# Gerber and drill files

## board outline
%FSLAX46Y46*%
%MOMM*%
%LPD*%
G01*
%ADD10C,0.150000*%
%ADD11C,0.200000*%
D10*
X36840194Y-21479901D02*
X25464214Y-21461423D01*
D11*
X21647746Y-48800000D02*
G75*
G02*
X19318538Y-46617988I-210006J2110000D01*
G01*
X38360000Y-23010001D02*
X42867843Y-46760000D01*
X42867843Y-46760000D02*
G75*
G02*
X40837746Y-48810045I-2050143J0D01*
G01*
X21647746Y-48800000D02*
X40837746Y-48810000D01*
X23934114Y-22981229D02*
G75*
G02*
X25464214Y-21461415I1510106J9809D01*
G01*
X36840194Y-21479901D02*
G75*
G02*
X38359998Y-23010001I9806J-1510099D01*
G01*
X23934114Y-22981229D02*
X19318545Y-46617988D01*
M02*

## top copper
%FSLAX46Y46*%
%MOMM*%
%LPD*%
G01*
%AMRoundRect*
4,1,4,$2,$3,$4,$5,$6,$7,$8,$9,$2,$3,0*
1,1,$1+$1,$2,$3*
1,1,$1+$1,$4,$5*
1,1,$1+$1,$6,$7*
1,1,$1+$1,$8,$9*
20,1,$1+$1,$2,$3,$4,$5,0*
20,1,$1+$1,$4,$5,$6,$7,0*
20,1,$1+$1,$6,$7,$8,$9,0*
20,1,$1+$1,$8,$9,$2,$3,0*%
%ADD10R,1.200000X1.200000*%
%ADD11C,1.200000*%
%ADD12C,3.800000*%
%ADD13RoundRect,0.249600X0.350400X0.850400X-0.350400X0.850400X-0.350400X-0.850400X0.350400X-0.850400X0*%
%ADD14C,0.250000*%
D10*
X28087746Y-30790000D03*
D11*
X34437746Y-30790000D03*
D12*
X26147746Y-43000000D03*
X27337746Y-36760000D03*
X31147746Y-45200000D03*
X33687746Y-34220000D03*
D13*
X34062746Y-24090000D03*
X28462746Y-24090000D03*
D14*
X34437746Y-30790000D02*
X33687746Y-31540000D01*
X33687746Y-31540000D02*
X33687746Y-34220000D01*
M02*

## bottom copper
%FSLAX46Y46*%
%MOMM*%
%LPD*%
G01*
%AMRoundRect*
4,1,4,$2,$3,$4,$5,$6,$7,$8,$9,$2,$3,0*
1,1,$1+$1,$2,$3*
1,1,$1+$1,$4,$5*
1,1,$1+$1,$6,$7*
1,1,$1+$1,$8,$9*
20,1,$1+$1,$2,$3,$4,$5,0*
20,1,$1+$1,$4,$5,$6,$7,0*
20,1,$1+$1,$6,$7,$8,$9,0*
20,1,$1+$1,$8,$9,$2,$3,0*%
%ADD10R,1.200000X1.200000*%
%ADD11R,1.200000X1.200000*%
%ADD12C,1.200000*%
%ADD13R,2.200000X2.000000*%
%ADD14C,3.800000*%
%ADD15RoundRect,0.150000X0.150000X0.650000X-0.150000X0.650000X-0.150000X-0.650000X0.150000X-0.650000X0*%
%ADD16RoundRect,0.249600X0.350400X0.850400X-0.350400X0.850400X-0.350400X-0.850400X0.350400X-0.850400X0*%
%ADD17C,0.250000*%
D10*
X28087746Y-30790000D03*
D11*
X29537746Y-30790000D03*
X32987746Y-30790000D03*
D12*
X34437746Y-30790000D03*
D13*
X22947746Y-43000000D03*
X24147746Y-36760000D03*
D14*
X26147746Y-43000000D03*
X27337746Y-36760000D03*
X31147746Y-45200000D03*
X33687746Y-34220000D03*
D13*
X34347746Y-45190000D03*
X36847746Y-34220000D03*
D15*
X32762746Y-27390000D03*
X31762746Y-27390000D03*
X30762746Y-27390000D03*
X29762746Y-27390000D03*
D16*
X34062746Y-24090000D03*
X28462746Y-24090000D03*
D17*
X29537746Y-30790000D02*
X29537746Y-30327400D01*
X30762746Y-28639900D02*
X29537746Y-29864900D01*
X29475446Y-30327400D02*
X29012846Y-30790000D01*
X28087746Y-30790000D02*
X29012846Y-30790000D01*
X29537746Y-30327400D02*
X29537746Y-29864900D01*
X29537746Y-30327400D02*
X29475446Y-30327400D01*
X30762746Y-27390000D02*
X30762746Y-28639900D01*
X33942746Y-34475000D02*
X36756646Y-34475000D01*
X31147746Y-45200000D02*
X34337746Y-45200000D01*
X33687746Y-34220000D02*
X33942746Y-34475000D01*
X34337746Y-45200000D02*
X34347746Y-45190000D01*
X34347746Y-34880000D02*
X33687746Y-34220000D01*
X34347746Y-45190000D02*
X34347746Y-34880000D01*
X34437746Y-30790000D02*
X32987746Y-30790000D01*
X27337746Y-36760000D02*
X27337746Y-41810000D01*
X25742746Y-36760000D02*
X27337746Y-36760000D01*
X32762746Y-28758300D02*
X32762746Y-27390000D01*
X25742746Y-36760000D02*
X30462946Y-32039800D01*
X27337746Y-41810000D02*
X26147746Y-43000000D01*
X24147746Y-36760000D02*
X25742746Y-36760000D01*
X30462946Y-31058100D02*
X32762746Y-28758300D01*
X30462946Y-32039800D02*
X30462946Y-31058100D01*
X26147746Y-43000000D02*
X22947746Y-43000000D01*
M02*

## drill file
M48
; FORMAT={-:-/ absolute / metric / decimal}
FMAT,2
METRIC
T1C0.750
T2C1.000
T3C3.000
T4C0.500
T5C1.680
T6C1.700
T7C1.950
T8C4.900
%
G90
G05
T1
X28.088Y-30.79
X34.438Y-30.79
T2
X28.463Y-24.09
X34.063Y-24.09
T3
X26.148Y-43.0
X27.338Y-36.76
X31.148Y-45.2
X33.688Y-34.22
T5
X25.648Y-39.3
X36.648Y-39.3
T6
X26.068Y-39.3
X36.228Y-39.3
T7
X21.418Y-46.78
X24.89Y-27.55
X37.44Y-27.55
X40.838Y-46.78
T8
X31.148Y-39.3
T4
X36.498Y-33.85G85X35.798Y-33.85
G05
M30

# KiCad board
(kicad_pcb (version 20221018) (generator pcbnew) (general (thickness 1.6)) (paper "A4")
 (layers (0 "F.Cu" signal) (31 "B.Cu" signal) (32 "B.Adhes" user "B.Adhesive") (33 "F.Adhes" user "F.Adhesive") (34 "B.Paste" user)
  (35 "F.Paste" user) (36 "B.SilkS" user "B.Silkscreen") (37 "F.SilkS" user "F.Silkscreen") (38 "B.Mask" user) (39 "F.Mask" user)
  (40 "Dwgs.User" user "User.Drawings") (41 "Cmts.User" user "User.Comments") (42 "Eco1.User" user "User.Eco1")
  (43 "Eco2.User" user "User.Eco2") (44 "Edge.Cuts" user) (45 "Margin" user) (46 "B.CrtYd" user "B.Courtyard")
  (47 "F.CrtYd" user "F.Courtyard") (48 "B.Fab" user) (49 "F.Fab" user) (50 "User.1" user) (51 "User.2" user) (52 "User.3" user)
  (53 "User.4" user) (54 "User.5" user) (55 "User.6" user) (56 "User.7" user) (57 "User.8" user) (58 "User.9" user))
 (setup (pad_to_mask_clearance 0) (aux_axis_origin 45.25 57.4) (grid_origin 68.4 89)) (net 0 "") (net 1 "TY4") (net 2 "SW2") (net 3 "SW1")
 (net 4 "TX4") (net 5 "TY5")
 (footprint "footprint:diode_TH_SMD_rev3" (layer "F.Cu") (at 31.262746 30.79)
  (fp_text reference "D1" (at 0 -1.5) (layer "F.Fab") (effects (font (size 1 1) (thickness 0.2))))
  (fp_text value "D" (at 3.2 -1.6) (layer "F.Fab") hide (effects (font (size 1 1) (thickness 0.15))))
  (pad "1" thru_hole rect (at -3.175 0) (size 1.2 1.2) (drill 0.75) (layers "*.Cu" "B.Mask") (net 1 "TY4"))
  (pad "1" smd rect (at -1.725 0) (size 1.2 1.2) (layers "B.Cu" "B.Paste" "B.Mask") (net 1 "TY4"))
  (pad "2" smd rect (at 1.725 0) (size 1.2 1.2) (layers "B.Cu" "B.Paste" "B.Mask") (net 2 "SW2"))
  (pad "2" thru_hole circle (at 3.175 0) (size 1.2 1.2) (drill 0.75) (layers "*.Cu" "B.Mask") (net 2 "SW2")))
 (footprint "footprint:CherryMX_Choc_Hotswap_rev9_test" (layer "F.Cu") (at 31.147746 39.3)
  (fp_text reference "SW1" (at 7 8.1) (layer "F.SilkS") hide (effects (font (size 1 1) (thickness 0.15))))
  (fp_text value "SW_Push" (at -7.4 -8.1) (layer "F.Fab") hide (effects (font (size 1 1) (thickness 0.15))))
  (pad "" np_thru_hole circle (at -5.5 0 90) (size 1.68 1.68) (drill 1.68) (layers "*.Cu" "*.Mask"))
  (pad "" np_thru_hole circle (at -5.08 0) (size 1.7 1.7) (drill 1.7) (layers "*.Cu" "*.Mask"))
  (pad "" np_thru_hole circle (at 0 0 90) (size 4.9 4.9) (drill 4.9) (layers "*.Cu" "*.Mask"))
  (pad "" np_thru_hole oval (at 5 -5.45 180) (size 1.2 0.5) (drill oval 1.2 0.5) (layers "*.Cu" "*.Mask"))
  (pad "" np_thru_hole circle (at 5.08 0) (size 1.7 1.7) (drill 1.7) (layers "*.Cu" "*.Mask"))
  (pad "" np_thru_hole circle (at 5.5 0 90) (size 1.68 1.68) (drill 1.68) (layers "*.Cu" "*.Mask"))
  (pad "1" smd rect (at -8.2 3.7) (size 2.2 2) (layers "B.Cu" "B.Paste" "B.Mask") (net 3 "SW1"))
  (pad "1" smd rect (at -7 -2.54) (size 2.2 2) (layers "B.Cu" "B.Paste" "B.Mask") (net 3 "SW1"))
  (pad "1" thru_hole circle (at -5 3.7 90) (size 3.8 3.8) (drill 3) (layers "*.Cu" "B.Mask") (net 3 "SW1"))
  (pad "1" thru_hole circle (at -3.81 -2.54 180) (size 3.8 3.8) (drill 3) (layers "*.Cu" "B.Mask") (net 3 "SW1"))
  (pad "2" thru_hole circle (at 0 5.9 90) (size 3.8 3.8) (drill 3) (layers "*.Cu" "B.Mask") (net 2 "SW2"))
  (pad "2" thru_hole circle (at 2.54 -5.08 180) (size 3.8 3.8) (drill 3) (layers "*.Cu" "B.Mask") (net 2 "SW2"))
  (pad "2" smd rect (at 3.2 5.89) (size 2.2 2) (layers "B.Cu" "B.Paste" "B.Mask") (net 2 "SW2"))
  (pad "2" smd rect (at 5.7 -5.08) (size 2.2 2) (layers "B.Cu" "B.Paste" "B.Mask") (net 2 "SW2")))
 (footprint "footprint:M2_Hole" (layer "F.Cu") (at 40.837746 46.78)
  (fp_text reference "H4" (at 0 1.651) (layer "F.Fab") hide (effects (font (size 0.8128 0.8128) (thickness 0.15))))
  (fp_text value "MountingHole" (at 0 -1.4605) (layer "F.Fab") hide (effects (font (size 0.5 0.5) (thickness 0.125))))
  (pad "" np_thru_hole circle (at 0 0) (size 1.95 1.95) (drill 1.95) (layers "F&B.Cu" "*.Mask")))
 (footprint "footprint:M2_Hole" (layer "F.Cu") (at 21.417746 46.78)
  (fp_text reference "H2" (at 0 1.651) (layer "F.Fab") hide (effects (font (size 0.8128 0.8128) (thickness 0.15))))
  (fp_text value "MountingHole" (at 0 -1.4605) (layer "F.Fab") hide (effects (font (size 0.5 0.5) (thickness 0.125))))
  (pad "" np_thru_hole circle (at 0 0) (size 1.95 1.95) (drill 1.95) (layers "F&B.Cu" "*.Mask")))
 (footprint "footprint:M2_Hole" (layer "F.Cu") (at 24.89 27.55)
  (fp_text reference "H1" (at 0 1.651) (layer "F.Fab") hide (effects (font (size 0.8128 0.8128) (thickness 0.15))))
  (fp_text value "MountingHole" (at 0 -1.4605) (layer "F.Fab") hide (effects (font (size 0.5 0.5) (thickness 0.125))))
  (pad "" np_thru_hole circle (at 0 0) (size 1.95 1.95) (drill 1.95) (layers "F&B.Cu" "*.Mask")))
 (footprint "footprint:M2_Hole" (layer "F.Cu") (at 37.44 27.55)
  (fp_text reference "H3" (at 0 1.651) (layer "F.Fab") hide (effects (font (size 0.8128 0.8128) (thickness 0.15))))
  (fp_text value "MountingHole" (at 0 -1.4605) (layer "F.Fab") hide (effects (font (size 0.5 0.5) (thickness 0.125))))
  (pad "" np_thru_hole circle (at 0 0) (size 1.95 1.95) (drill 1.95) (layers "F&B.Cu" "*.Mask")))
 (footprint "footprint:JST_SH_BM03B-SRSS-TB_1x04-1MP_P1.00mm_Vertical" (layer "B.Cu") (at 31.262746 25.59 180)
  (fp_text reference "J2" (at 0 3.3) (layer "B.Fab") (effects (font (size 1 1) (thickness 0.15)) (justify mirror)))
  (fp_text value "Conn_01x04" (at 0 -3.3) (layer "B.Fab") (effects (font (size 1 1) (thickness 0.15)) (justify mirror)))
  (pad "1" smd roundrect (at -1.5 -1.8 180) (size 0.6 1.6) (layers "B.Cu" "B.Paste" "B.Mask") (roundrect_rratio 0.25) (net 3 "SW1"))
  (pad "2" smd roundrect (at -0.5 -1.8 180) (size 0.6 1.6) (layers "B.Cu" "B.Paste" "B.Mask") (roundrect_rratio 0.25) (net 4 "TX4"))
  (pad "3" smd roundrect (at 0.5 -1.8 180) (size 0.6 1.6) (layers "B.Cu" "B.Paste" "B.Mask") (roundrect_rratio 0.25) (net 1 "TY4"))
  (pad "4" smd roundrect (at 1.5 -1.8 180) (size 0.6 1.6) (layers "B.Cu" "B.Paste" "B.Mask") (roundrect_rratio 0.25) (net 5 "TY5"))
  (pad "MP" thru_hole roundrect (at -2.8 1.5 180) (size 1.2 2.2) (drill 1) (layers "*.Cu" "*.Mask") (roundrect_rratio 0.208))
  (pad "MP" thru_hole roundrect (at 2.8 1.5 180) (size 1.2 2.2) (drill 1) (layers "*.Cu" "*.Mask") (roundrect_rratio 0.208)))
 (gr_line (start 36.840194 21.479901) (end 25.464214 21.461423) (stroke (width 0.15) (type default)) (layer "Edge.Cuts"))
 (gr_arc (start 21.647746 48.8) (mid 19.988071 48.237464) (end 19.318545 46.617988) (stroke (width 0.2) (type default)) (layer "Edge.Cuts"))
 (gr_line (start 38.36 23.010001) (end 42.867843 46.76) (stroke (width 0.2) (type default)) (layer "Edge.Cuts"))
 (gr_arc (start 42.867843 46.76) (mid 42.274437 48.202549) (end 40.837746 48.809999) (stroke (width 0.2) (type default)) (layer "Edge.Cuts"))
 (gr_line (start 21.647746 48.8) (end 40.837746 48.81) (stroke (width 0.2) (type default)) (layer "Edge.Cuts"))
 (gr_arc (start 23.934114 22.981229) (mid 24.38 21.900001) (end 25.464214 21.461423) (stroke (width 0.2) (type default)) (layer "Edge.Cuts"))
 (gr_arc (start 36.840194 21.479901) (mid 37.921422 21.925787) (end 38.36 23.010001) (stroke (width 0.2) (type default)) (layer "Edge.Cuts"))
 (gr_line (start 23.934114 22.981229) (end 19.318545 46.617988) (stroke (width 0.2) (type default)) (layer "Edge.Cuts"))
 (segment (start 29.537746 30.79) (end 29.537746 30.3274) (width 0.25) (layer "B.Cu") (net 1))
 (segment (start 30.762746 28.6399) (end 29.537746 29.8649) (width 0.25) (layer "B.Cu") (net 1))
 (segment (start 29.475446 30.3274) (end 29.012846 30.79) (width 0.25) (layer "B.Cu") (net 1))
 (segment (start 28.087746 30.79) (end 29.012846 30.79) (width 0.25) (layer "B.Cu") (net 1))
 (segment (start 29.537746 30.3274) (end 29.537746 29.8649) (width 0.25) (layer "B.Cu") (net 1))
 (segment (start 29.537746 30.3274) (end 29.475446 30.3274) (width 0.25) (layer "B.Cu") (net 1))
 (segment (start 30.762746 27.39) (end 30.762746 28.6399) (width 0.25) (layer "B.Cu") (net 1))
 (segment (start 34.437746 30.79) (end 33.687746 31.54) (width 0.25) (layer "F.Cu") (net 2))
 (segment (start 33.687746 31.54) (end 33.687746 34.22) (width 0.25) (layer "F.Cu") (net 2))
 (segment (start 33.942746 34.475) (end 36.756646 34.475) (width 0.25) (layer "B.Cu") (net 2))
 (segment (start 31.147746 45.2) (end 34.337746 45.2) (width 0.25) (layer "B.Cu") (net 2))
 (segment (start 33.687746 34.22) (end 33.942746 34.475) (width 0.25) (layer "B.Cu") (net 2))
 (segment (start 34.337746 45.2) (end 34.347746 45.19) (width 0.25) (layer "B.Cu") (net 2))
 (segment (start 34.347746 34.88) (end 33.687746 34.22) (width 0.25) (layer "B.Cu") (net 2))
 (segment (start 34.347746 45.19) (end 34.347746 34.88) (width 0.25) (layer "B.Cu") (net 2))
 (segment (start 34.437746 30.79) (end 32.987746 30.79) (width 0.25) (layer "B.Cu") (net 2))
 (segment (start 27.337746 36.76) (end 27.337746 41.81) (width 0.25) (layer "B.Cu") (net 3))
 (segment (start 25.742746 36.76) (end 27.337746 36.76) (width 0.25) (layer "B.Cu") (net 3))
 (segment (start 32.762746 28.7583) (end 32.762746 27.39) (width 0.25) (layer "B.Cu") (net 3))
 (segment (start 25.742746 36.76) (end 30.462946 32.0398) (width 0.25) (layer "B.Cu") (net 3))
 (segment (start 27.337746 41.81) (end 26.147746 43) (width 0.25) (layer "B.Cu") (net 3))
 (segment (start 24.147746 36.76) (end 25.742746 36.76) (width 0.25) (layer "B.Cu") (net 3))
 (segment (start 30.462946 31.0581) (end 32.762746 28.7583) (width 0.25) (layer "B.Cu") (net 3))
 (segment (start 30.462946 32.0398) (end 30.462946 31.0581) (width 0.25) (layer "B.Cu") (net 3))
 (segment (start 26.147746 43) (end 22.947746 43) (width 0.25) (layer "B.Cu") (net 3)))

